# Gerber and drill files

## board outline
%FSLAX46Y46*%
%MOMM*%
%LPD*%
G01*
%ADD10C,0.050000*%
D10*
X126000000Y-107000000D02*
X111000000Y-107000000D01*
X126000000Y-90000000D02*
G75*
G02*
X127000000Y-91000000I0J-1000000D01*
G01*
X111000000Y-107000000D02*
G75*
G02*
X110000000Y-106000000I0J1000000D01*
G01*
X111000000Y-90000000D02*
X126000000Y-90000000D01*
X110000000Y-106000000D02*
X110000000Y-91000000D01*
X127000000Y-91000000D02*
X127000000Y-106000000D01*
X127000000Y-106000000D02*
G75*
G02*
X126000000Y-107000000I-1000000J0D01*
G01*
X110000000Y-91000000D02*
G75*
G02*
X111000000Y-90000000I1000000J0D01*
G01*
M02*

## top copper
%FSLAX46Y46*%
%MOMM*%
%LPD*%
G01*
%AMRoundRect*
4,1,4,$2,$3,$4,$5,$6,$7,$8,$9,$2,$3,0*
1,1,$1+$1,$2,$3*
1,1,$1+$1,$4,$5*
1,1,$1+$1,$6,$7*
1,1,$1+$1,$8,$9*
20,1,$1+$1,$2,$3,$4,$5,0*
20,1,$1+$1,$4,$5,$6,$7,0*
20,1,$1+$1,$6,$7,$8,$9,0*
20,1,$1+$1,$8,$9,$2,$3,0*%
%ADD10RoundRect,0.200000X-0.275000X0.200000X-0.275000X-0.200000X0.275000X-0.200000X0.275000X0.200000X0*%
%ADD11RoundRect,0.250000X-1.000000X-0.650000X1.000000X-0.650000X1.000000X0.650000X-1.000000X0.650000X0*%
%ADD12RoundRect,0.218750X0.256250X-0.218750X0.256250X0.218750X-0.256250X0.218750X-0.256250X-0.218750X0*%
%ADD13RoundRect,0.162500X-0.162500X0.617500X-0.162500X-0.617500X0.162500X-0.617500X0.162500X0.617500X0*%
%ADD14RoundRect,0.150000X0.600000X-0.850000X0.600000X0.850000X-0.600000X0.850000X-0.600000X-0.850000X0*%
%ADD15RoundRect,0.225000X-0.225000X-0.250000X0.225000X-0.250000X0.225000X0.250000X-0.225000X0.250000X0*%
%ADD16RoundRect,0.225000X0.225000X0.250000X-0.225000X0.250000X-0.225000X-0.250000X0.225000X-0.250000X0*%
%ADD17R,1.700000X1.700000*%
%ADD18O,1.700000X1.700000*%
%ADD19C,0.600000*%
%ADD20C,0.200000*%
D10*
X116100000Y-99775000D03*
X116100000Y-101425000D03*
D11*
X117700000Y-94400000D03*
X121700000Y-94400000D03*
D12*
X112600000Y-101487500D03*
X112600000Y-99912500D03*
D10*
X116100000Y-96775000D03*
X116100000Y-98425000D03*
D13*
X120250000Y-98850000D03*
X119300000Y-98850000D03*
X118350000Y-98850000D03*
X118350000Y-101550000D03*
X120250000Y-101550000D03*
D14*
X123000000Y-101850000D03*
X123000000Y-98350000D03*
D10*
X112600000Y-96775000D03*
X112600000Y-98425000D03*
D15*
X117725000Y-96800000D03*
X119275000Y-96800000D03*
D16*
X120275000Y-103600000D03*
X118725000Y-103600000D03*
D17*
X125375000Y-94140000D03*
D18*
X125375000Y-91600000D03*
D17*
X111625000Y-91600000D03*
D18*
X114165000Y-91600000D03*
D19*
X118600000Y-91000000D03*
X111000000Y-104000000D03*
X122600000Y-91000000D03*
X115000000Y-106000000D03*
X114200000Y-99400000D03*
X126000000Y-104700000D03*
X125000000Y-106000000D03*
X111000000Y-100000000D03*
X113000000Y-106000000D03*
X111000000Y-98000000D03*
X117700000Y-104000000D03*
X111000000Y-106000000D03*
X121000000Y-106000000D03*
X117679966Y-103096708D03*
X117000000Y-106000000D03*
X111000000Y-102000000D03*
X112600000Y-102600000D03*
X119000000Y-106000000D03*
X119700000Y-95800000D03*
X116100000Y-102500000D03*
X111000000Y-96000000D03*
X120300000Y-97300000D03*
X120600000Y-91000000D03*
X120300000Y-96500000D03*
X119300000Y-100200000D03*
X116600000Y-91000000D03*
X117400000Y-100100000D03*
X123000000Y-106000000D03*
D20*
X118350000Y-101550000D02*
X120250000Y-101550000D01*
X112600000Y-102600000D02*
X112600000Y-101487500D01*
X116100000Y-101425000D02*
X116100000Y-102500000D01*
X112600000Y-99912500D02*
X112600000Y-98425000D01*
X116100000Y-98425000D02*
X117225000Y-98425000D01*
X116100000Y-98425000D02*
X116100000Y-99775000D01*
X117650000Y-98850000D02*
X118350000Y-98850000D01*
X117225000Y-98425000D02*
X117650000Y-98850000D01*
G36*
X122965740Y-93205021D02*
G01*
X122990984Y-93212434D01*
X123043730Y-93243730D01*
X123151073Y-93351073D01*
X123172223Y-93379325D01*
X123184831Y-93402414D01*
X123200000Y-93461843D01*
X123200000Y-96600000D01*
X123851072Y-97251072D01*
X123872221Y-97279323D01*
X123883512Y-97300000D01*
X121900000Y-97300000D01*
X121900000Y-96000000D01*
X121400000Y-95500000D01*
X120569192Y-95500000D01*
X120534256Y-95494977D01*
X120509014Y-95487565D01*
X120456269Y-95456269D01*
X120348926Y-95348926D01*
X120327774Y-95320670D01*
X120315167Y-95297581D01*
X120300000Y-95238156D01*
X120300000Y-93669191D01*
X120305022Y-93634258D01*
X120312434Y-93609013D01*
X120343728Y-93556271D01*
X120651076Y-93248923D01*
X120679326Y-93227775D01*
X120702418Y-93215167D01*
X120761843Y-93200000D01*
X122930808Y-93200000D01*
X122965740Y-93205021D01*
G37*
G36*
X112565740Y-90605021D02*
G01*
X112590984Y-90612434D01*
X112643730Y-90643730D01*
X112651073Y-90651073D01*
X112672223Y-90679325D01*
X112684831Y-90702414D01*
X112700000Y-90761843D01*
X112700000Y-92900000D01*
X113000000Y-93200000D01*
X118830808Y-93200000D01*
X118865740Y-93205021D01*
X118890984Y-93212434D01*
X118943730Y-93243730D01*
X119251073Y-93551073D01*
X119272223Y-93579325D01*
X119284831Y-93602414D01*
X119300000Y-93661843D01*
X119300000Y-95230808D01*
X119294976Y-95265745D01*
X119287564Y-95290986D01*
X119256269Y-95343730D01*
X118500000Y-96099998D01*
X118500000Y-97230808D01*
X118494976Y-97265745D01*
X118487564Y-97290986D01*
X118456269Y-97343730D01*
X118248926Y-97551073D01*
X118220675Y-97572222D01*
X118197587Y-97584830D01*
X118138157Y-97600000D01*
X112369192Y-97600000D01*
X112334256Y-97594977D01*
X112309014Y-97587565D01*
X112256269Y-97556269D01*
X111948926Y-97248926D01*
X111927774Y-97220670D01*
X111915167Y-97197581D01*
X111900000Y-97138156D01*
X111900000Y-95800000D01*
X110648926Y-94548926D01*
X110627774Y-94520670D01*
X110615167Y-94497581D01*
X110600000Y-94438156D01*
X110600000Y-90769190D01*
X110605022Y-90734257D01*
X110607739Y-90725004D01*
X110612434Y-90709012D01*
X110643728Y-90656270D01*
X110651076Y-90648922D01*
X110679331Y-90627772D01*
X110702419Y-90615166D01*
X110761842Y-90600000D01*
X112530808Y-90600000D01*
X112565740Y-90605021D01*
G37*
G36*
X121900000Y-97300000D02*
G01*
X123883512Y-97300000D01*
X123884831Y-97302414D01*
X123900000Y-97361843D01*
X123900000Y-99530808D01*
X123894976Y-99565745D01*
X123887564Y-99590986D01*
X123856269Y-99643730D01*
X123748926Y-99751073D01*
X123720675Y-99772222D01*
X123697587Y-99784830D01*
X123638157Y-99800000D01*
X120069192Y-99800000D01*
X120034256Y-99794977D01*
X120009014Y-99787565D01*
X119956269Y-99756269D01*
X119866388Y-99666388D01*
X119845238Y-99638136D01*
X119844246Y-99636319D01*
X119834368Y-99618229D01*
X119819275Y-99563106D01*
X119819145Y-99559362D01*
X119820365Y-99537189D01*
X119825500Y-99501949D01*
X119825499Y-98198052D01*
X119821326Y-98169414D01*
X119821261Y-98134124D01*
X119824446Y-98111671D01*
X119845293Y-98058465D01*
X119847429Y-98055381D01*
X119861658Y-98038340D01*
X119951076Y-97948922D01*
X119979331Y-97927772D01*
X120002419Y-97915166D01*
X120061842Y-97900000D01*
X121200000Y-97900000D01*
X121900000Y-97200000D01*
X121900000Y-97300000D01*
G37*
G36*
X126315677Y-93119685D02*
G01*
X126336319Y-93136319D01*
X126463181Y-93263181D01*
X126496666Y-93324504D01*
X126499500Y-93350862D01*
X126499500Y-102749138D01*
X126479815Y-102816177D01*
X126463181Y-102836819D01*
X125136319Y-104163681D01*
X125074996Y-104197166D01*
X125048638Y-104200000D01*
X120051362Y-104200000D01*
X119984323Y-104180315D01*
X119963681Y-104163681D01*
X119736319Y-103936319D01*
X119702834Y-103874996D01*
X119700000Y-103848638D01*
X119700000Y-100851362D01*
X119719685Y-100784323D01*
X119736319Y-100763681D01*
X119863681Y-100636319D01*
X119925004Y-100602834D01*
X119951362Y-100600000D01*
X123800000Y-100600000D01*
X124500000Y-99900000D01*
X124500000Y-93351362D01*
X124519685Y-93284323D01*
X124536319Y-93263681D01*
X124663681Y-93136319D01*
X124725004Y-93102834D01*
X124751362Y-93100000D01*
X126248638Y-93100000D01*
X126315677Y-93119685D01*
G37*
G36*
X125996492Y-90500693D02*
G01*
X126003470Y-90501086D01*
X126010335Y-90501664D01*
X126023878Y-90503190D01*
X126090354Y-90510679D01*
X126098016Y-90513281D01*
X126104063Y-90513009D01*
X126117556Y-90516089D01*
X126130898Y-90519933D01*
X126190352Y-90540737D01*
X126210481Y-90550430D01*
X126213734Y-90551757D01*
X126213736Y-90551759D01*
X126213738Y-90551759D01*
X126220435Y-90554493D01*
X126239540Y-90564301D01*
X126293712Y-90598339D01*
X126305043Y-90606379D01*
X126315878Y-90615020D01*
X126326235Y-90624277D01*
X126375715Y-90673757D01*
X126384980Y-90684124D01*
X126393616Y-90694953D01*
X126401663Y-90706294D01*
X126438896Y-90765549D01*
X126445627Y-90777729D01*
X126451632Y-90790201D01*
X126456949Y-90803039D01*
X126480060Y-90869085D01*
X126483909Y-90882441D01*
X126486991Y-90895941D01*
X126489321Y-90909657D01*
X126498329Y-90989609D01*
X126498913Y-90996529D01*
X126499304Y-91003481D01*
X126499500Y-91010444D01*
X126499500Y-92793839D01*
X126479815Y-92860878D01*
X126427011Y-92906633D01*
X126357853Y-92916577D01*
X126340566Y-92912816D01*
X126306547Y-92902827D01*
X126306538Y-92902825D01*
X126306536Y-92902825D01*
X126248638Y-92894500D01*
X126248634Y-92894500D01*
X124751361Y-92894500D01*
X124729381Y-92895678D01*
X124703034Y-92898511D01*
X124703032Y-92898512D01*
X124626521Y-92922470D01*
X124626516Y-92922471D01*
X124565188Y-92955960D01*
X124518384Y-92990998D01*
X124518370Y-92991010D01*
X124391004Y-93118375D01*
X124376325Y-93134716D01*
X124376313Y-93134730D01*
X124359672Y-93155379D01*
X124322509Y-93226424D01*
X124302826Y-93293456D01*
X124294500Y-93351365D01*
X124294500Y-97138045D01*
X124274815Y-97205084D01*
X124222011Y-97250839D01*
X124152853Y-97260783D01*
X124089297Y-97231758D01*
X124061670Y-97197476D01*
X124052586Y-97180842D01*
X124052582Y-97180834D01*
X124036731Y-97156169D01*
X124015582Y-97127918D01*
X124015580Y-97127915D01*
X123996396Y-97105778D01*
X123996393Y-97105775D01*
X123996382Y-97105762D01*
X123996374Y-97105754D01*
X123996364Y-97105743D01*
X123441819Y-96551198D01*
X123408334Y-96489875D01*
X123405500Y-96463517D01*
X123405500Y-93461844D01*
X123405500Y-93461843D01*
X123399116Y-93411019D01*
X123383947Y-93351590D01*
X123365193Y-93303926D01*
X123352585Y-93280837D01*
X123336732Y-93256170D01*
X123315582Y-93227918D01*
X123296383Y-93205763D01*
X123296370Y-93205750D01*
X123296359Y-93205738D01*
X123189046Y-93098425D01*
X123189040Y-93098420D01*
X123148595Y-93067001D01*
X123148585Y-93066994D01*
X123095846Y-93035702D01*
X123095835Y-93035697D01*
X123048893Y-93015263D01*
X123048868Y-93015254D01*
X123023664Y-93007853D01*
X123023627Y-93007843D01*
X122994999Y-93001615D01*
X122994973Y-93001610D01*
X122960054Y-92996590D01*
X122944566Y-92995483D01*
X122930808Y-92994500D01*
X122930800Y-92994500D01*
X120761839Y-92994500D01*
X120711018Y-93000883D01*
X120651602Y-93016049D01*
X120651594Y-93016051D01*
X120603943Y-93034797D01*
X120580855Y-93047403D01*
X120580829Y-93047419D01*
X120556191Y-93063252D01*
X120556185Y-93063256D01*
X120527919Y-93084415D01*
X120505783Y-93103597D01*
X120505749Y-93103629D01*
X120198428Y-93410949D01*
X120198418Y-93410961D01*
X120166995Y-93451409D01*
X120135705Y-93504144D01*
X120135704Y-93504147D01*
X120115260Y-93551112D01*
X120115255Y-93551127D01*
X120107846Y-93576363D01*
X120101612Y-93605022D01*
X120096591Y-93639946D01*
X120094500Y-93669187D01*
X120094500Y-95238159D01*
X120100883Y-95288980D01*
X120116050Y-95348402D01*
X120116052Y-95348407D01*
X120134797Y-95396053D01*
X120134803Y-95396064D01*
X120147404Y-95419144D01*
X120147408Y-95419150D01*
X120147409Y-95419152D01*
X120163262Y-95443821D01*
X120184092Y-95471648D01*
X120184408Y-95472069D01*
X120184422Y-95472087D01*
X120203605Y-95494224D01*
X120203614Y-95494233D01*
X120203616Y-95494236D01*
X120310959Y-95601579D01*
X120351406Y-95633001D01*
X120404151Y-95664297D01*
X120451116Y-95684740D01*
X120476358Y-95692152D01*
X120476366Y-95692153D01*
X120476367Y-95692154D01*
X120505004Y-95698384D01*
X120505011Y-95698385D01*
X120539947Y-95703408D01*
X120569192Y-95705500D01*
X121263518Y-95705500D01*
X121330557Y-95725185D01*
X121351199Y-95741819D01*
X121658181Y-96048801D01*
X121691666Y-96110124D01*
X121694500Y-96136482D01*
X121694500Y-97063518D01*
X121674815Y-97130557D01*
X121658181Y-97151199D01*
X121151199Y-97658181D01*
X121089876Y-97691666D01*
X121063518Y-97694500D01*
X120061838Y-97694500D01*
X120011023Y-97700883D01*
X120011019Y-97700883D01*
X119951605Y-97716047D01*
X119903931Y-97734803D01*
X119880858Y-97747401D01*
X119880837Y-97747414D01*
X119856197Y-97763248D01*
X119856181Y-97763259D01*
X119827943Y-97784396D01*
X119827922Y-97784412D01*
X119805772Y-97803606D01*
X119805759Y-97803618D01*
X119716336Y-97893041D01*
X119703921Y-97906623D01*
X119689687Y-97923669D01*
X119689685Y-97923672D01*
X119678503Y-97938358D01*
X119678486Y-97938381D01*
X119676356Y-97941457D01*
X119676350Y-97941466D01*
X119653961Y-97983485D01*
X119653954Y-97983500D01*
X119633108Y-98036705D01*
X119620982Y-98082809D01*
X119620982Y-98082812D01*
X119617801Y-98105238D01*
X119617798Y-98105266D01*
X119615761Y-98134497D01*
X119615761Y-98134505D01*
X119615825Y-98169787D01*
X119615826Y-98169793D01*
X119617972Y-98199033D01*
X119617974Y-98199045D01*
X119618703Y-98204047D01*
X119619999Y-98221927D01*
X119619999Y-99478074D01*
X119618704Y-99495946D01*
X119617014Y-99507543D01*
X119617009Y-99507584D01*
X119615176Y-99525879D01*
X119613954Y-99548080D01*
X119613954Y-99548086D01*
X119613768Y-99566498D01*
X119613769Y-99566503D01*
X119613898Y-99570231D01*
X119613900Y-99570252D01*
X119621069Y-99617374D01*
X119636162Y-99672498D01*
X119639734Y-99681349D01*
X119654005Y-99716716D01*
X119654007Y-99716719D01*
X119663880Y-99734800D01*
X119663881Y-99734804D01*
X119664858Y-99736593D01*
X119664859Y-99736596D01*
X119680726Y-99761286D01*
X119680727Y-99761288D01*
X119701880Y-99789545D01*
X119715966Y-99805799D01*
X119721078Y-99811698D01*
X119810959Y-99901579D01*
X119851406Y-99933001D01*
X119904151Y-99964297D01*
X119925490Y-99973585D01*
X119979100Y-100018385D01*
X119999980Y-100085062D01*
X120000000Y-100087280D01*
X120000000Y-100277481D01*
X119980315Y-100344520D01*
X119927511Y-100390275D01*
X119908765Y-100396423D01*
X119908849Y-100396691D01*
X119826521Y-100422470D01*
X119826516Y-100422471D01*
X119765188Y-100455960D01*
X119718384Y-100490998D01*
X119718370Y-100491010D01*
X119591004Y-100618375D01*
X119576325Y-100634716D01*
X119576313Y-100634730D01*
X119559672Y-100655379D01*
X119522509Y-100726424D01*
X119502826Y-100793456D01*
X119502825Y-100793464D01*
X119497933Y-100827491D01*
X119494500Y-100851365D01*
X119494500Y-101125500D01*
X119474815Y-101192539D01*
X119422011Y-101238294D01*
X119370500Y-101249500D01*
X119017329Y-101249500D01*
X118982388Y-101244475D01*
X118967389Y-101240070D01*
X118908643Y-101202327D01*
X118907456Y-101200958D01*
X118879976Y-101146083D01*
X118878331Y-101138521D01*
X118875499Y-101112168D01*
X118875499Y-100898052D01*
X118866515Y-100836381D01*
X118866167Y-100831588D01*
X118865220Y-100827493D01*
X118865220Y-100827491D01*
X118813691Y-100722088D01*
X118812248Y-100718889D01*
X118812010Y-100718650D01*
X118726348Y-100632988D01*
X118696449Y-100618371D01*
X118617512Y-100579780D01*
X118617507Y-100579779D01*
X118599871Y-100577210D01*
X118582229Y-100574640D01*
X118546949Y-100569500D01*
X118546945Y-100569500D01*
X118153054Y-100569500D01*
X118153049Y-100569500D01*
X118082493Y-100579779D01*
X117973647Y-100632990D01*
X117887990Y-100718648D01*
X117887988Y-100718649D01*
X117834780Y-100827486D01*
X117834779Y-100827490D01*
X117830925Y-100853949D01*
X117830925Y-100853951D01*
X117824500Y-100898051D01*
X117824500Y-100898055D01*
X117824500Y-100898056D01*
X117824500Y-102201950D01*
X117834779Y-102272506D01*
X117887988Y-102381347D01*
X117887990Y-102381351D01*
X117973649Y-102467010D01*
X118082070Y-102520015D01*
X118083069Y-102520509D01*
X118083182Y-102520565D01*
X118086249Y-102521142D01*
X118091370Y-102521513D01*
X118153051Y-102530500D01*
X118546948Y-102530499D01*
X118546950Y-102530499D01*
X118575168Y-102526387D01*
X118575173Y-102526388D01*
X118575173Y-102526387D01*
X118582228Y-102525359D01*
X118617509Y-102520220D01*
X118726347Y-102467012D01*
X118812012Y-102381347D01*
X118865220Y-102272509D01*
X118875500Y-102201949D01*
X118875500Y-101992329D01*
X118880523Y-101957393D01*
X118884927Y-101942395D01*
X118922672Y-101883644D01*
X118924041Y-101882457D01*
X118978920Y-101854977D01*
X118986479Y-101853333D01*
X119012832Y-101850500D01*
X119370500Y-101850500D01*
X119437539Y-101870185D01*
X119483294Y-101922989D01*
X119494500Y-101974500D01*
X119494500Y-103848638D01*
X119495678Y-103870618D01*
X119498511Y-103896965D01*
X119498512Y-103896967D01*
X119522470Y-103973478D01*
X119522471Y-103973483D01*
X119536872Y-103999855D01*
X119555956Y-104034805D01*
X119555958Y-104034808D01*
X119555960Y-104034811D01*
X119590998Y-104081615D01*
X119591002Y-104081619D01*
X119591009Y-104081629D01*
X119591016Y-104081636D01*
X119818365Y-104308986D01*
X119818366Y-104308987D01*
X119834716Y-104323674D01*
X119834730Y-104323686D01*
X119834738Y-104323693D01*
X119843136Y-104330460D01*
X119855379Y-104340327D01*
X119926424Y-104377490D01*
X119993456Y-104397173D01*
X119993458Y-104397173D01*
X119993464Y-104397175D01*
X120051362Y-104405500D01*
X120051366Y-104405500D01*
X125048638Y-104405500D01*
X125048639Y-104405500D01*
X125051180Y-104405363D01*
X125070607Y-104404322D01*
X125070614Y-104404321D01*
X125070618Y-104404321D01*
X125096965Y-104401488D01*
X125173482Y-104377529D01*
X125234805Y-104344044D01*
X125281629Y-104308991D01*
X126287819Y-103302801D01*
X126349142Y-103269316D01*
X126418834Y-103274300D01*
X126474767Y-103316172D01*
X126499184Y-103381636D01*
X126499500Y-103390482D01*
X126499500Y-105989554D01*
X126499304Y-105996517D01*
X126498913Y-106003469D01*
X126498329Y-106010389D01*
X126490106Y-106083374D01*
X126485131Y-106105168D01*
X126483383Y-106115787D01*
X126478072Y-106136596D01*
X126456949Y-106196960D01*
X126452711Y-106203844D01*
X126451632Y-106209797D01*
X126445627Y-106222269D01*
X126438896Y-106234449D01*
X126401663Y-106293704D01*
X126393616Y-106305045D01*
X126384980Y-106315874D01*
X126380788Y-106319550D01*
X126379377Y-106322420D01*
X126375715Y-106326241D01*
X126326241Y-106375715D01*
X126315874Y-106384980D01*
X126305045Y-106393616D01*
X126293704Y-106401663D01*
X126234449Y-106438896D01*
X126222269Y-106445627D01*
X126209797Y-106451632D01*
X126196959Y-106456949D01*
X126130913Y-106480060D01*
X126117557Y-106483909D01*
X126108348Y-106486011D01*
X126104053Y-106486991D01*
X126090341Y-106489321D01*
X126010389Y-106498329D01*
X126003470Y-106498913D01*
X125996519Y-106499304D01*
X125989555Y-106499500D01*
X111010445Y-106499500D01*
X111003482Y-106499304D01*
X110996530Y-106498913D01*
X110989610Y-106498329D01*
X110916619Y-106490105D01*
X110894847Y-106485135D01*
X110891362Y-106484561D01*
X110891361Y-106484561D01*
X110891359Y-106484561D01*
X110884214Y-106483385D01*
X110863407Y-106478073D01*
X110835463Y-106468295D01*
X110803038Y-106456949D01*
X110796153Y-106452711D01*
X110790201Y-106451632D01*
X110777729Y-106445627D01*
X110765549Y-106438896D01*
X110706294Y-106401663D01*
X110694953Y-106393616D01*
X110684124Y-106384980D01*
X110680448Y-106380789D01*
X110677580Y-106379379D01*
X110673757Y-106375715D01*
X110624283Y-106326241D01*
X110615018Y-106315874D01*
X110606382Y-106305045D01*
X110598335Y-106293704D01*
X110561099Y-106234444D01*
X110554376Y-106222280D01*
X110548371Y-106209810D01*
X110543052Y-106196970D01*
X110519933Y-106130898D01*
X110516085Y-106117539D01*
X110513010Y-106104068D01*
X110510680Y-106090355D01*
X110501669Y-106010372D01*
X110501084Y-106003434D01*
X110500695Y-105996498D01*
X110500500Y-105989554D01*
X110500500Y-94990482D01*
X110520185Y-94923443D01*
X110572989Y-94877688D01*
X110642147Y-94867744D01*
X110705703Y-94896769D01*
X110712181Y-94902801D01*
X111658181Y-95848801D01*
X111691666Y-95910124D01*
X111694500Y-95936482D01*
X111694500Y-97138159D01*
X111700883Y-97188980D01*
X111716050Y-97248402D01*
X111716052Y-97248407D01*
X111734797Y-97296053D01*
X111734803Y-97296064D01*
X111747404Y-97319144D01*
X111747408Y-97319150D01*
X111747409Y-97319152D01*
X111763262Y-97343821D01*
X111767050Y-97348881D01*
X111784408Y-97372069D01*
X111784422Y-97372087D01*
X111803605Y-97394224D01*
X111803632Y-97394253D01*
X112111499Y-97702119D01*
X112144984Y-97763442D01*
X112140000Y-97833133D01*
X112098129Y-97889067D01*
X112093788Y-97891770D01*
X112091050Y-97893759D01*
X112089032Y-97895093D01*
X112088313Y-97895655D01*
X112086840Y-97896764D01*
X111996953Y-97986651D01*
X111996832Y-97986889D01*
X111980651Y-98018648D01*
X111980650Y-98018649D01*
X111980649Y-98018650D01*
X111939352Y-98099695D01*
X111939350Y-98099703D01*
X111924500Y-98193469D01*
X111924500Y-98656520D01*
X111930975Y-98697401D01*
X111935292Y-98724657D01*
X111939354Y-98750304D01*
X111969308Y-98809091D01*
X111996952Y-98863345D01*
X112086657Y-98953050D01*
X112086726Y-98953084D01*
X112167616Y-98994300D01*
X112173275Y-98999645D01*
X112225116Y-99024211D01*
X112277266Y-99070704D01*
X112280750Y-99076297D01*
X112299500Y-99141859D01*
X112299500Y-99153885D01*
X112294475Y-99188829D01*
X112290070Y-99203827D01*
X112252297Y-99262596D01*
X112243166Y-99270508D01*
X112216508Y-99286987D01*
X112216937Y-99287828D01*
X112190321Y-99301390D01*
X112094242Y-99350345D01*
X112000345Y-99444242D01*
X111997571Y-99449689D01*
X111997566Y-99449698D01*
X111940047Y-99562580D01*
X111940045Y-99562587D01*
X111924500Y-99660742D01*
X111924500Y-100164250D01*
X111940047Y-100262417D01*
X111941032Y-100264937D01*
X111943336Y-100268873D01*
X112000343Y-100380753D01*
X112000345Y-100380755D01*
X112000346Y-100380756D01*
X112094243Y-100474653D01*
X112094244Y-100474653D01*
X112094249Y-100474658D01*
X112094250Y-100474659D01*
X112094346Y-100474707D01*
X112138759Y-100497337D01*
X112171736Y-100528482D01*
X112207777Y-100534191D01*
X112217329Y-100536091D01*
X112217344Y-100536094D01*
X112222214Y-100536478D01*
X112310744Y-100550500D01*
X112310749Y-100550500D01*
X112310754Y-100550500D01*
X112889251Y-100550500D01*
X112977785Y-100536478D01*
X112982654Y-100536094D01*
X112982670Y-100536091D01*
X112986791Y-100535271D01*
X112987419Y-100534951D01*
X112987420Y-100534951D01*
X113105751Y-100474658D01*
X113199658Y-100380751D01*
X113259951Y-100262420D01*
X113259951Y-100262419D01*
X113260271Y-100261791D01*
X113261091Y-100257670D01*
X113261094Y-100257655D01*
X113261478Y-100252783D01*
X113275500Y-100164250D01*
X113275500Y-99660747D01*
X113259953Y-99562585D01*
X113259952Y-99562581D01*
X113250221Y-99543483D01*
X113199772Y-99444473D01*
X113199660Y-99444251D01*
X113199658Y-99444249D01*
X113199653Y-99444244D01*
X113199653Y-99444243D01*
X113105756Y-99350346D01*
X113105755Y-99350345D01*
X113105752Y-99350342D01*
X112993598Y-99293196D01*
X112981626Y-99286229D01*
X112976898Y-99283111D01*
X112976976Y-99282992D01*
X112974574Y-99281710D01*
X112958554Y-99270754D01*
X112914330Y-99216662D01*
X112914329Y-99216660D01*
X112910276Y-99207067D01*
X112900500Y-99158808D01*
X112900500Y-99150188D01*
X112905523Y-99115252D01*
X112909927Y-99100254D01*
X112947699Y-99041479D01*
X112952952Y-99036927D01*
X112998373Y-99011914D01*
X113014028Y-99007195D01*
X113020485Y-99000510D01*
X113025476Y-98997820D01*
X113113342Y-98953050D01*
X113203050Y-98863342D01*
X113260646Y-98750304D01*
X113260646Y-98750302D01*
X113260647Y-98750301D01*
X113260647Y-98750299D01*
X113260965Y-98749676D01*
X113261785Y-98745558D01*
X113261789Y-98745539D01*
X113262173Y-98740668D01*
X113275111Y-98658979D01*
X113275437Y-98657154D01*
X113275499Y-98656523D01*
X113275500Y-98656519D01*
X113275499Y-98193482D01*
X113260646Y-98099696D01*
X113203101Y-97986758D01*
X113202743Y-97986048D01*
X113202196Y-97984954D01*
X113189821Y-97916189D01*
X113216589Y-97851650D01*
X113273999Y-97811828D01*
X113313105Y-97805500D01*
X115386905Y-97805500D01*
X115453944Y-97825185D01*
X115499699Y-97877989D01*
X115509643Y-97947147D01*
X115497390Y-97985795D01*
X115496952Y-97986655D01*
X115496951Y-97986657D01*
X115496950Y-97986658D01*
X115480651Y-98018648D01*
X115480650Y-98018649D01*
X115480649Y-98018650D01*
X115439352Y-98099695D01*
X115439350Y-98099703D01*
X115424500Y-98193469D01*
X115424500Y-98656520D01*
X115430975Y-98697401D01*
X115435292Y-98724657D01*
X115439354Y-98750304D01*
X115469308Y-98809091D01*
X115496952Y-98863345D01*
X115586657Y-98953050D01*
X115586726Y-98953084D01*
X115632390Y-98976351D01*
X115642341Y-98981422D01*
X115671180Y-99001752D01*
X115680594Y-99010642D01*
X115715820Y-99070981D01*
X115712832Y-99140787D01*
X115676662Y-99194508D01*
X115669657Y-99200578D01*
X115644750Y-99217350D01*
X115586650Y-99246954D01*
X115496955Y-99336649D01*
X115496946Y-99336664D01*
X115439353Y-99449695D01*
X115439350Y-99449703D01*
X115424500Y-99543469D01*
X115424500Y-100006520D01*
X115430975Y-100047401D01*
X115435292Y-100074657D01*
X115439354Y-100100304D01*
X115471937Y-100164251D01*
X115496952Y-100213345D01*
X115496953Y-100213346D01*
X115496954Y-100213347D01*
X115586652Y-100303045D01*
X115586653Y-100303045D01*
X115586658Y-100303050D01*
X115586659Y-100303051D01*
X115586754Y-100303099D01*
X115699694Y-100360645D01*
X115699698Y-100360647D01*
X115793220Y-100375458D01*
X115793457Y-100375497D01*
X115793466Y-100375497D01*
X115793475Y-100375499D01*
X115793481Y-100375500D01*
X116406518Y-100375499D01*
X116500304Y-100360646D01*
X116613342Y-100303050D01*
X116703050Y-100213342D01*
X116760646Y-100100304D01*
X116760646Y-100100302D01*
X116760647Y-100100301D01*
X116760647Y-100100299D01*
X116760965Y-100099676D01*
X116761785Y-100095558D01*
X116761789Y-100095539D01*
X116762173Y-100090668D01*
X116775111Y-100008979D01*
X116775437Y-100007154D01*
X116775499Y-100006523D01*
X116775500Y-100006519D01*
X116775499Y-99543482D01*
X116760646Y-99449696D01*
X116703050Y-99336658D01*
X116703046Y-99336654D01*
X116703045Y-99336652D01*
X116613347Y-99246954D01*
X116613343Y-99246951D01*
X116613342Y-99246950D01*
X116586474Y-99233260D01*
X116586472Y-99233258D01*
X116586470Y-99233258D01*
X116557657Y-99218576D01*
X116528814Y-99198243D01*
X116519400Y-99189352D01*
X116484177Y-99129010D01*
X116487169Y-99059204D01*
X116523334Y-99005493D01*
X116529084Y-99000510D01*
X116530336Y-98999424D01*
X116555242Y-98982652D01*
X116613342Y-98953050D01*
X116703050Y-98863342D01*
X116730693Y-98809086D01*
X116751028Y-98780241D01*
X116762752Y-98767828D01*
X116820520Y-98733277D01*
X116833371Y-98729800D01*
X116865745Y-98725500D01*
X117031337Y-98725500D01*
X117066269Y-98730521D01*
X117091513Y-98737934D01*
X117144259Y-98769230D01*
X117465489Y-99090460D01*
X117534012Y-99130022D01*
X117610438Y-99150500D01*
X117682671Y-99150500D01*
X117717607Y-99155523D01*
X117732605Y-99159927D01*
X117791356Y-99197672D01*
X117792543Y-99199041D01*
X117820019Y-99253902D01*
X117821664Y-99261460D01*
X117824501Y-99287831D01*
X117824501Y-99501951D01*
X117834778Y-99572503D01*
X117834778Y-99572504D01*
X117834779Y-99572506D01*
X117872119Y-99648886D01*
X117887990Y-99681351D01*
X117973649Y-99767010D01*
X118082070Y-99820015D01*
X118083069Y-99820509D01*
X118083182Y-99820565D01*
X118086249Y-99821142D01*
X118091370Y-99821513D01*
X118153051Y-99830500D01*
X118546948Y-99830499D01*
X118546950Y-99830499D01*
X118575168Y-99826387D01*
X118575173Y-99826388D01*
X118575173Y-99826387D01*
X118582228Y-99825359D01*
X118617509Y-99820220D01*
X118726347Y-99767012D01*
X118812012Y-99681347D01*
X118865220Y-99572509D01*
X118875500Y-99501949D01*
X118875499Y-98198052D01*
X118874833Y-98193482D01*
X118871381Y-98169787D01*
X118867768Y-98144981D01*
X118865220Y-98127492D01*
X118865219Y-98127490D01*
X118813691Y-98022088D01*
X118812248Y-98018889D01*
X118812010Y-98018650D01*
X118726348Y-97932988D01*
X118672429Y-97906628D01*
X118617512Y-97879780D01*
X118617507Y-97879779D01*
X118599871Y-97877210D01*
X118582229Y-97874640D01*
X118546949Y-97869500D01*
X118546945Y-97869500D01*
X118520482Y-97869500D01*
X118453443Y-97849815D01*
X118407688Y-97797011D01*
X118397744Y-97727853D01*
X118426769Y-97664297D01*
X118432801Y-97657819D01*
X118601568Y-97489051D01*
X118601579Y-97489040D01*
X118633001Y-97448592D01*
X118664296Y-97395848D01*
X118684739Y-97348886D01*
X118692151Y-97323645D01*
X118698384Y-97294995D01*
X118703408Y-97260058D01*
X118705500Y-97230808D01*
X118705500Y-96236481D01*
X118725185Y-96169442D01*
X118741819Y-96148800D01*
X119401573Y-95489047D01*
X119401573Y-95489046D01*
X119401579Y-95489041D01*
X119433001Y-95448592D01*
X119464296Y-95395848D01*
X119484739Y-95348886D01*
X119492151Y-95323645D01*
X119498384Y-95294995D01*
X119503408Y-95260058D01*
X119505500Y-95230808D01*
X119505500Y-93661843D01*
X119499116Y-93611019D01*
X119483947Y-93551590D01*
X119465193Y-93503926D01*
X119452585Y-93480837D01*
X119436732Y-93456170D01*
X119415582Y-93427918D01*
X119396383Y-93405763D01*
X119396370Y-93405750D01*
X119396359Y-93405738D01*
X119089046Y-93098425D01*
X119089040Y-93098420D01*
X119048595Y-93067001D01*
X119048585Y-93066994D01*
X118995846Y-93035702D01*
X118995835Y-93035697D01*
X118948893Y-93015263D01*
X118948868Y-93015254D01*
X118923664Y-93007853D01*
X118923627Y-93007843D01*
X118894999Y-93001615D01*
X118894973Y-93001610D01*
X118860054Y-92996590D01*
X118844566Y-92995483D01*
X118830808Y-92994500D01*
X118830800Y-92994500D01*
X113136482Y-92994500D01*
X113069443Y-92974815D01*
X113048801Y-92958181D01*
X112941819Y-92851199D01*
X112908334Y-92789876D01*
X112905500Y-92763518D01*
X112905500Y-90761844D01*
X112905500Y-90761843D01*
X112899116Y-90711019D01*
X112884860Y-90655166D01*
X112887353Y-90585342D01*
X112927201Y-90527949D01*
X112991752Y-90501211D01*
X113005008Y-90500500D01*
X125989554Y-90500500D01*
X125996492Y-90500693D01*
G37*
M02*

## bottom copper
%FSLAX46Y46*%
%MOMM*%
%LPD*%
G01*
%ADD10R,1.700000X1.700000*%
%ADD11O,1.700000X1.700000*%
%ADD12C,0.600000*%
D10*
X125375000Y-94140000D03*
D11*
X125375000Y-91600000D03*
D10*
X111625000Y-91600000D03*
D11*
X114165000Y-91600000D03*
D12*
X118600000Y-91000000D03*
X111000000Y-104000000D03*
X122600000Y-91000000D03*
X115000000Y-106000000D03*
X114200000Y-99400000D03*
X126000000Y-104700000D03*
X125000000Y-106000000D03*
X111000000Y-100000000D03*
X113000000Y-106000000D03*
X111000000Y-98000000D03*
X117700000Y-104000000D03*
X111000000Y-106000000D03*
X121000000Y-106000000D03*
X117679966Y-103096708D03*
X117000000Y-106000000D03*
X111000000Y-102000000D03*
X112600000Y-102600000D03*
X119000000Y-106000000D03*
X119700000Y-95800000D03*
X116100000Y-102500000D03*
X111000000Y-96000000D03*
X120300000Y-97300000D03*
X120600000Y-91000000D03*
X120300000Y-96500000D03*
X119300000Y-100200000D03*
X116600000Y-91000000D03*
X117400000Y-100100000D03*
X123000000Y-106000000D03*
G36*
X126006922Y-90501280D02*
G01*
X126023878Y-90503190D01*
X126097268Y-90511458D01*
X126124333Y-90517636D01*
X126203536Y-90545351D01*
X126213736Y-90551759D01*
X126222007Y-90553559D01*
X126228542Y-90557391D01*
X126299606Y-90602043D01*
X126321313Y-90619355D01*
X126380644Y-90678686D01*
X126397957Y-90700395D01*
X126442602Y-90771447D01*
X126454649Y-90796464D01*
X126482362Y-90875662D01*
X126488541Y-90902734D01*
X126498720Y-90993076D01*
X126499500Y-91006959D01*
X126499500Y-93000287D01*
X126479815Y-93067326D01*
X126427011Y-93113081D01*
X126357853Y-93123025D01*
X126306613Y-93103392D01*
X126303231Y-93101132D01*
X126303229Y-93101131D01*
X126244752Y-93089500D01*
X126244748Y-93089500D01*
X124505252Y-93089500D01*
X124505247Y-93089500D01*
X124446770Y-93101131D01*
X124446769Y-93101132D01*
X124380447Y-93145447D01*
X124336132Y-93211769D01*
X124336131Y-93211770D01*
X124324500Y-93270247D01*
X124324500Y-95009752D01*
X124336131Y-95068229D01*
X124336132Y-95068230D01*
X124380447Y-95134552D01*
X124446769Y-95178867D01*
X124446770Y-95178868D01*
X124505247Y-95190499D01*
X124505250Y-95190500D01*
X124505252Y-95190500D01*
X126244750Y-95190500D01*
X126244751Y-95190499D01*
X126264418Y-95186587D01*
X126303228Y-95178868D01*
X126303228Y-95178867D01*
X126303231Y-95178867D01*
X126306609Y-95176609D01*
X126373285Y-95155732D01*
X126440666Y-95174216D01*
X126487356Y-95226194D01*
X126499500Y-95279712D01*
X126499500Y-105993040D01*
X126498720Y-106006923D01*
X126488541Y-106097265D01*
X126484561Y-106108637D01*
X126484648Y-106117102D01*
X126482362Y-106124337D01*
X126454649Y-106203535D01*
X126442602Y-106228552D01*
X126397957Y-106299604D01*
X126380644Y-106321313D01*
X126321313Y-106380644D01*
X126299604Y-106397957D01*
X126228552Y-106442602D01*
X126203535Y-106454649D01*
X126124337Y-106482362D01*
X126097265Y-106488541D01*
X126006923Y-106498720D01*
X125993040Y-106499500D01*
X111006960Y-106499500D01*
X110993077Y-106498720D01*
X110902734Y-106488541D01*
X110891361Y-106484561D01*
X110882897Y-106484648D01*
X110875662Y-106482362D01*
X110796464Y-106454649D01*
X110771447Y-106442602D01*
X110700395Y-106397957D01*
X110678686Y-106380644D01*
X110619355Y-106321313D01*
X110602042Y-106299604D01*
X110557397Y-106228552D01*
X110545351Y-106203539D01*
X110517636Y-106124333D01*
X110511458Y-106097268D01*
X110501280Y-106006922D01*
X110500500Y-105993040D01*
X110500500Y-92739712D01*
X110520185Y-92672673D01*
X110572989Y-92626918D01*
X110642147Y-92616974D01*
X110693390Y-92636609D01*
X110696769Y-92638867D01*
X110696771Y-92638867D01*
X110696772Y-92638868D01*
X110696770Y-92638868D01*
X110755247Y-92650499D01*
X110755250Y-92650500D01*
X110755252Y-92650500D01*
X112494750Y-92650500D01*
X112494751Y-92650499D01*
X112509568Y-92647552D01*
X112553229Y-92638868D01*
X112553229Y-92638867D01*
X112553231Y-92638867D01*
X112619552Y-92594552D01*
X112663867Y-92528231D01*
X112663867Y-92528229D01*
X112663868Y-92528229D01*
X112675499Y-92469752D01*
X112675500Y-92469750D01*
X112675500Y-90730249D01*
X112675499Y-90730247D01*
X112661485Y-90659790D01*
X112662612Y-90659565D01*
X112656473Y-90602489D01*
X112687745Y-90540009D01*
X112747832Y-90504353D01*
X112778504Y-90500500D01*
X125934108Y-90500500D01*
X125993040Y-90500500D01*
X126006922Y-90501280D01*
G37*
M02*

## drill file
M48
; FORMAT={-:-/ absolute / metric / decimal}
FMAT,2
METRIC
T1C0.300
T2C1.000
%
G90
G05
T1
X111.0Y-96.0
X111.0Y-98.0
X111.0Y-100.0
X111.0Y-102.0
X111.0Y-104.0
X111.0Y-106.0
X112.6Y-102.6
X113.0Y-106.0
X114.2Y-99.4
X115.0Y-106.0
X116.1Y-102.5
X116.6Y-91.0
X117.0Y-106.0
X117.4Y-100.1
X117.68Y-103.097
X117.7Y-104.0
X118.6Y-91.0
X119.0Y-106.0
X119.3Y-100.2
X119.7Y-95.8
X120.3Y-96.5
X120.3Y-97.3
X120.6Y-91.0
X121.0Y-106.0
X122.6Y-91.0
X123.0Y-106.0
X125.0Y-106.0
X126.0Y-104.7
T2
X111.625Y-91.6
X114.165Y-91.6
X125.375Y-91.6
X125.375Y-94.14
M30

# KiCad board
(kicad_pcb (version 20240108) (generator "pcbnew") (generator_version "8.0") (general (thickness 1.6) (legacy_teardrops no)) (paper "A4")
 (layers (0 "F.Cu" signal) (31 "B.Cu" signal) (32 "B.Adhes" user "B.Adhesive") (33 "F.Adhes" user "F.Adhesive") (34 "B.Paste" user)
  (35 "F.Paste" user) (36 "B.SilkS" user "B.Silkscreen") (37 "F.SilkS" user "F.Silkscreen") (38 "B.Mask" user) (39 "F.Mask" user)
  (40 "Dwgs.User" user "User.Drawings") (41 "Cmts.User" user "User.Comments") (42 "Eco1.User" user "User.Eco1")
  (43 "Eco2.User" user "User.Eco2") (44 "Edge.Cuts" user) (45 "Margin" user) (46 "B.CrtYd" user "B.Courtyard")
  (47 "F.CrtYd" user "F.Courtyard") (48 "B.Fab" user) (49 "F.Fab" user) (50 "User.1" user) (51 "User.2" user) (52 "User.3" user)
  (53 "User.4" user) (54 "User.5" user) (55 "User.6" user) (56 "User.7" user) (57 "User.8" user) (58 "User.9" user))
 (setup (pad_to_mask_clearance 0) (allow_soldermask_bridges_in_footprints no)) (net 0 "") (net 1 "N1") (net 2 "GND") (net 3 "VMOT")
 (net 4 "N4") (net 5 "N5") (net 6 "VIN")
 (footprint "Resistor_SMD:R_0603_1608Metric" (layer "F.Cu") (at 116.1 100.6 -90)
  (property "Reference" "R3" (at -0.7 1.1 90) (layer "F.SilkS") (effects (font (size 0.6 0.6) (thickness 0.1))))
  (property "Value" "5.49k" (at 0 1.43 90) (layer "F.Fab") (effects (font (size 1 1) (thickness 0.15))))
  (pad "1" smd roundrect (at -0.825 0 270) (size 0.8 0.95) (layers "F.Cu" "F.Paste" "F.Mask") (roundrect_rratio 0.25) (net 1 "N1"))
  (pad "2" smd roundrect (at 0.825 0 270) (size 0.8 0.95) (layers "F.Cu" "F.Paste" "F.Mask") (roundrect_rratio 0.25) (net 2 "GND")))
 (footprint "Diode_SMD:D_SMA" (layer "F.Cu") (at 119.7 94.4)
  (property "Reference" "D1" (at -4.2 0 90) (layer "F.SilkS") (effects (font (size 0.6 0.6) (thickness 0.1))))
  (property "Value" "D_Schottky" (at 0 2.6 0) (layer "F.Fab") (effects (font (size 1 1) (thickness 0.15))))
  (pad "1" smd roundrect (at -2 0) (size 2.5 1.8) (layers "F.Cu" "F.Paste" "F.Mask") (roundrect_rratio 0.1388888889) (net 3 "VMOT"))
  (pad "2" smd roundrect (at 2 0) (size 2.5 1.8) (layers "F.Cu" "F.Paste" "F.Mask") (roundrect_rratio 0.1388888889) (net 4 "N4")))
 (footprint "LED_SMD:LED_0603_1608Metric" (layer "F.Cu") (at 112.6 100.7 90)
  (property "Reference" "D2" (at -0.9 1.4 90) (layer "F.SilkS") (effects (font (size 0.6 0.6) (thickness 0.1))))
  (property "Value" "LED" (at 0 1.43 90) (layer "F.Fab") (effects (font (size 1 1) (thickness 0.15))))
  (pad "1" smd roundrect (at -0.7875 0 90) (size 0.875 0.95) (layers "F.Cu" "F.Paste" "F.Mask") (roundrect_rratio 0.25) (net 2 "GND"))
  (pad "2" smd roundrect (at 0.7875 0 90) (size 0.875 0.95) (layers "F.Cu" "F.Paste" "F.Mask") (roundrect_rratio 0.25) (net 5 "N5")))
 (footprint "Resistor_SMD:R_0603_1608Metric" (layer "F.Cu") (at 116.1 97.6 -90)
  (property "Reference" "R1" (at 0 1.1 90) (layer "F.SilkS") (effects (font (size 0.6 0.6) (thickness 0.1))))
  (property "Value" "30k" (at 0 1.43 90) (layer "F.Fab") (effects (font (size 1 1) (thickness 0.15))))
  (pad "1" smd roundrect (at -0.825 0 270) (size 0.8 0.95) (layers "F.Cu" "F.Paste" "F.Mask") (roundrect_rratio 0.25) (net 3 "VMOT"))
  (pad "2" smd roundrect (at 0.825 0 270) (size 0.8 0.95) (layers "F.Cu" "F.Paste" "F.Mask") (roundrect_rratio 0.25) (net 1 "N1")))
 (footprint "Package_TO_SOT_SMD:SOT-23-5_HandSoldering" (layer "F.Cu") (at 119.3 100.2 -90)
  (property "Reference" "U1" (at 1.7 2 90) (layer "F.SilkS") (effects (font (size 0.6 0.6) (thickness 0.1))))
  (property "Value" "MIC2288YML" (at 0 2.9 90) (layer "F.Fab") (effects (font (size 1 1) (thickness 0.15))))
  (pad "1" smd roundrect (at -1.35 -0.95 270) (size 1.56 0.65) (layers "F.Cu" "F.Paste" "F.Mask") (roundrect_rratio 0.25) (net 4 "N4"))
  (pad "2" smd roundrect (at -1.35 0 270) (size 1.56 0.65) (layers "F.Cu" "F.Paste" "F.Mask") (roundrect_rratio 0.25) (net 2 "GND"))
  (pad "3" smd roundrect (at -1.35 0.95 270) (size 1.56 0.65) (layers "F.Cu" "F.Paste" "F.Mask") (roundrect_rratio 0.25) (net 1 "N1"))
  (pad "4" smd roundrect (at 1.35 0.95 270) (size 1.56 0.65) (layers "F.Cu" "F.Paste" "F.Mask") (roundrect_rratio 0.25) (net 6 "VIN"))
  (pad "5" smd roundrect (at 1.35 -0.95 270) (size 1.56 0.65) (layers "F.Cu" "F.Paste" "F.Mask") (roundrect_rratio 0.25) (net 6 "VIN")))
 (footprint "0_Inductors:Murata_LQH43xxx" (layer "F.Cu") (at 123 100.1 90)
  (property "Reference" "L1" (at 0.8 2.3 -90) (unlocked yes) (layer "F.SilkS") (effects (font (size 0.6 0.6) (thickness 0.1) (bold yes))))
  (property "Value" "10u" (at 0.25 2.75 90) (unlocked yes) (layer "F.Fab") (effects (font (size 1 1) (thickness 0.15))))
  (pad "1" smd roundrect (at -1.75 0 90) (size 2 1.5) (layers "F.Cu" "F.Paste" "F.Mask") (roundrect_rratio 0.1) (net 6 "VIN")
   (thermal_bridge_angle 45))
  (pad "2" smd roundrect (at 1.75 0 90) (size 2 1.5) (layers "F.Cu" "F.Paste" "F.Mask") (roundrect_rratio 0.1) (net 4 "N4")
   (thermal_bridge_angle 45)))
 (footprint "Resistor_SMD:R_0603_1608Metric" (layer "F.Cu") (at 112.6 97.6 -90)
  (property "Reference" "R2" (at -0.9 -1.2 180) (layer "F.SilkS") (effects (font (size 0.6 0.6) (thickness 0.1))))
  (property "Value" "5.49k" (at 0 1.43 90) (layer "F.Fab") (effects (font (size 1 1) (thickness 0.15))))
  (pad "1" smd roundrect (at -0.825 0 270) (size 0.8 0.95) (layers "F.Cu" "F.Paste" "F.Mask") (roundrect_rratio 0.25) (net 3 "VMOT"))
  (pad "2" smd roundrect (at 0.825 0 270) (size 0.8 0.95) (layers "F.Cu" "F.Paste" "F.Mask") (roundrect_rratio 0.25) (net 5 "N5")))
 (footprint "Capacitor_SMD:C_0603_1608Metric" (layer "F.Cu") (at 118.5 96.8)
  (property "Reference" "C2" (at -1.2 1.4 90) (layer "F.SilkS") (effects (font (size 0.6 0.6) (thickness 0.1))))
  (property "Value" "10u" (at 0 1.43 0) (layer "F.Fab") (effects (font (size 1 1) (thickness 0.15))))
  (pad "1" smd roundrect (at -0.775 0) (size 0.9 0.95) (layers "F.Cu" "F.Paste" "F.Mask") (roundrect_rratio 0.25) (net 3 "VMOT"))
  (pad "2" smd roundrect (at 0.775 0) (size 0.9 0.95) (layers "F.Cu" "F.Paste" "F.Mask") (roundrect_rratio 0.25) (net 2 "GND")))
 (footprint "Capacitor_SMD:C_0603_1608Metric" (layer "F.Cu") (at 119.5 103.6 180)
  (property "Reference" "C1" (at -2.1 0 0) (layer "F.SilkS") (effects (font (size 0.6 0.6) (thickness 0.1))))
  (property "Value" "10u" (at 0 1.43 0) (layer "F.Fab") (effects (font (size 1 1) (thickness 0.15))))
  (pad "1" smd roundrect (at -0.775 0 180) (size 0.9 0.95) (layers "F.Cu" "F.Paste" "F.Mask") (roundrect_rratio 0.25) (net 6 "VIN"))
  (pad "2" smd roundrect (at 0.775 0 180) (size 0.9 0.95) (layers "F.Cu" "F.Paste" "F.Mask") (roundrect_rratio 0.25) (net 2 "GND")))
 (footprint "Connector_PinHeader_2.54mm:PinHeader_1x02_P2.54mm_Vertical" (layer "B.Cu") (at 125.375 94.14)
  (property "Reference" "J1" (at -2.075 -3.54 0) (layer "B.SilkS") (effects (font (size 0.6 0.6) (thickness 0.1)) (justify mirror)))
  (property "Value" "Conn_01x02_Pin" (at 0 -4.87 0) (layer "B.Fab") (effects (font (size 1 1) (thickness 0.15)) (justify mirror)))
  (pad "1" thru_hole rect (at 0 0) (size 1.7 1.7) (drill 1) (layers "*.Cu" "*.Mask") (remove_unused_layers no) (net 6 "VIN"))
  (pad "2" thru_hole oval (at 0 -2.54) (size 1.7 1.7) (drill 1) (layers "*.Cu" "*.Mask") (remove_unused_layers no) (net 2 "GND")))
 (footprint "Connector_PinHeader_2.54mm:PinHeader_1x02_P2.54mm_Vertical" (layer "B.Cu") (at 111.625 91.6 -90)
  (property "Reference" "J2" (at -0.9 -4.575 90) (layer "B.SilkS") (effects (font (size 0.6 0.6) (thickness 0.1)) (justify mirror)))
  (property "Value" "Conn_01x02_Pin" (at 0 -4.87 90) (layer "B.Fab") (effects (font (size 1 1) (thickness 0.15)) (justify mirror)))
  (pad "1" thru_hole rect (at 0 0 270) (size 1.7 1.7) (drill 1) (layers "*.Cu" "*.Mask") (remove_unused_layers no) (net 3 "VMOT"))
  (pad "2" thru_hole oval (at 0 -2.54 270) (size 1.7 1.7) (drill 1) (layers "*.Cu" "*.Mask") (remove_unused_layers no) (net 2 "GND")))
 (gr_line (start 126 107) (end 111 107) (stroke (width 0.05) (type default)) (layer "Edge.Cuts"))
 (gr_arc (start 126 90) (mid 126.707107 90.292893) (end 127 91) (stroke (width 0.05) (type default)) (layer "Edge.Cuts"))
 (gr_arc (start 111 107) (mid 110.292893 106.707107) (end 110 106) (stroke (width 0.05) (type default)) (layer "Edge.Cuts"))
 (gr_line (start 111 90) (end 126 90) (stroke (width 0.05) (type default)) (layer "Edge.Cuts"))
 (gr_line (start 110 106) (end 110 91) (stroke (width 0.05) (type default)) (layer "Edge.Cuts"))
 (gr_line (start 127 91) (end 127 106) (stroke (width 0.05) (type default)) (layer "Edge.Cuts"))
 (gr_arc (start 127 106) (mid 126.707107 106.707107) (end 126 107) (stroke (width 0.05) (type default)) (layer "Edge.Cuts"))
 (gr_arc (start 110 91) (mid 110.292893 90.292893) (end 111 90) (stroke (width 0.05) (type default)) (layer "Edge.Cuts"))
 (segment (start 118.35 101.55) (end 120.25 101.55) (width 0.2) (layer "F.Cu") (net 6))
 (segment (start 112.6 102.6) (end 112.6 101.4875) (width 0.2) (layer "F.Cu") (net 2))
 (segment (start 116.1 101.425) (end 116.1 102.5) (width 0.2) (layer "F.Cu") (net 2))
 (via (at 118.6 91) (size 0.6) (drill 0.3) (layers "F.Cu" "B.Cu") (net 2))
 (via (at 111 104) (size 0.6) (drill 0.3) (layers "F.Cu" "B.Cu") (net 2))
 (via (at 122.6 91) (size 0.6) (drill 0.3) (layers "F.Cu" "B.Cu") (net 2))
 (via (at 115 106) (size 0.6) (drill 0.3) (layers "F.Cu" "B.Cu") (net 2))
 (via (at 114.2 99.4) (size 0.6) (drill 0.3) (layers "F.Cu" "B.Cu") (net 2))
 (via (at 126 104.7) (size 0.6) (drill 0.3) (layers "F.Cu" "B.Cu") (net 2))
 (via (at 125 106) (size 0.6) (drill 0.3) (layers "F.Cu" "B.Cu") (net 2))
 (via (at 111 100) (size 0.6) (drill 0.3) (layers "F.Cu" "B.Cu") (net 2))
 (via (at 113 106) (size 0.6) (drill 0.3) (layers "F.Cu" "B.Cu") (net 2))
 (via (at 111 98) (size 0.6) (drill 0.3) (layers "F.Cu" "B.Cu") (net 2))
 (via (at 117.7 104) (size 0.6) (drill 0.3) (layers "F.Cu" "B.Cu") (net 2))
 (via (at 111 106) (size 0.6) (drill 0.3) (layers "F.Cu" "B.Cu") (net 2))
 (via (at 121 106) (size 0.6) (drill 0.3) (layers "F.Cu" "B.Cu") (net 2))
 (via (at 117.679966 103.096708) (size 0.6) (drill 0.3) (layers "F.Cu" "B.Cu") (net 2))
 (via (at 117 106) (size 0.6) (drill 0.3) (layers "F.Cu" "B.Cu") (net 2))
 (via (at 111 102) (size 0.6) (drill 0.3) (layers "F.Cu" "B.Cu") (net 2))
 (via (at 112.6 102.6) (size 0.6) (drill 0.3) (layers "F.Cu" "B.Cu") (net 2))
 (via (at 119 106) (size 0.6) (drill 0.3) (layers "F.Cu" "B.Cu") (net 2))
 (via (at 119.7 95.8) (size 0.6) (drill 0.3) (layers "F.Cu" "B.Cu") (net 2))
 (via (at 116.1 102.5) (size 0.6) (drill 0.3) (layers "F.Cu" "B.Cu") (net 2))
 (via (at 111 96) (size 0.6) (drill 0.3) (layers "F.Cu" "B.Cu") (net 2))
 (via (at 120.3 97.3) (size 0.6) (drill 0.3) (layers "F.Cu" "B.Cu") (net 2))
 (via (at 120.6 91) (size 0.6) (drill 0.3) (layers "F.Cu" "B.Cu") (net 2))
 (via (at 120.3 96.5) (size 0.6) (drill 0.3) (layers "F.Cu" "B.Cu") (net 2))
 (via (at 119.3 100.2) (size 0.6) (drill 0.3) (layers "F.Cu" "B.Cu") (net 2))
 (via (at 116.6 91) (size 0.6) (drill 0.3) (layers "F.Cu" "B.Cu") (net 2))
 (via (at 117.4 100.1) (size 0.6) (drill 0.3) (layers "F.Cu" "B.Cu") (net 2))
 (via (at 123 106) (size 0.6) (drill 0.3) (layers "F.Cu" "B.Cu") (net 2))
 (segment (start 112.6 99.9125) (end 112.6 98.425) (width 0.2) (layer "F.Cu") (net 5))
 (segment (start 116.1 98.425) (end 117.225 98.425) (width 0.2) (layer "F.Cu") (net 1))
 (segment (start 116.1 98.425) (end 116.1 99.775) (width 0.2) (layer "F.Cu") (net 1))
 (segment (start 117.65 98.85) (end 118.35 98.85) (width 0.2) (layer "F.Cu") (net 1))
 (segment (start 117.225 98.425) (end 117.65 98.85) (width 0.2) (layer "F.Cu") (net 1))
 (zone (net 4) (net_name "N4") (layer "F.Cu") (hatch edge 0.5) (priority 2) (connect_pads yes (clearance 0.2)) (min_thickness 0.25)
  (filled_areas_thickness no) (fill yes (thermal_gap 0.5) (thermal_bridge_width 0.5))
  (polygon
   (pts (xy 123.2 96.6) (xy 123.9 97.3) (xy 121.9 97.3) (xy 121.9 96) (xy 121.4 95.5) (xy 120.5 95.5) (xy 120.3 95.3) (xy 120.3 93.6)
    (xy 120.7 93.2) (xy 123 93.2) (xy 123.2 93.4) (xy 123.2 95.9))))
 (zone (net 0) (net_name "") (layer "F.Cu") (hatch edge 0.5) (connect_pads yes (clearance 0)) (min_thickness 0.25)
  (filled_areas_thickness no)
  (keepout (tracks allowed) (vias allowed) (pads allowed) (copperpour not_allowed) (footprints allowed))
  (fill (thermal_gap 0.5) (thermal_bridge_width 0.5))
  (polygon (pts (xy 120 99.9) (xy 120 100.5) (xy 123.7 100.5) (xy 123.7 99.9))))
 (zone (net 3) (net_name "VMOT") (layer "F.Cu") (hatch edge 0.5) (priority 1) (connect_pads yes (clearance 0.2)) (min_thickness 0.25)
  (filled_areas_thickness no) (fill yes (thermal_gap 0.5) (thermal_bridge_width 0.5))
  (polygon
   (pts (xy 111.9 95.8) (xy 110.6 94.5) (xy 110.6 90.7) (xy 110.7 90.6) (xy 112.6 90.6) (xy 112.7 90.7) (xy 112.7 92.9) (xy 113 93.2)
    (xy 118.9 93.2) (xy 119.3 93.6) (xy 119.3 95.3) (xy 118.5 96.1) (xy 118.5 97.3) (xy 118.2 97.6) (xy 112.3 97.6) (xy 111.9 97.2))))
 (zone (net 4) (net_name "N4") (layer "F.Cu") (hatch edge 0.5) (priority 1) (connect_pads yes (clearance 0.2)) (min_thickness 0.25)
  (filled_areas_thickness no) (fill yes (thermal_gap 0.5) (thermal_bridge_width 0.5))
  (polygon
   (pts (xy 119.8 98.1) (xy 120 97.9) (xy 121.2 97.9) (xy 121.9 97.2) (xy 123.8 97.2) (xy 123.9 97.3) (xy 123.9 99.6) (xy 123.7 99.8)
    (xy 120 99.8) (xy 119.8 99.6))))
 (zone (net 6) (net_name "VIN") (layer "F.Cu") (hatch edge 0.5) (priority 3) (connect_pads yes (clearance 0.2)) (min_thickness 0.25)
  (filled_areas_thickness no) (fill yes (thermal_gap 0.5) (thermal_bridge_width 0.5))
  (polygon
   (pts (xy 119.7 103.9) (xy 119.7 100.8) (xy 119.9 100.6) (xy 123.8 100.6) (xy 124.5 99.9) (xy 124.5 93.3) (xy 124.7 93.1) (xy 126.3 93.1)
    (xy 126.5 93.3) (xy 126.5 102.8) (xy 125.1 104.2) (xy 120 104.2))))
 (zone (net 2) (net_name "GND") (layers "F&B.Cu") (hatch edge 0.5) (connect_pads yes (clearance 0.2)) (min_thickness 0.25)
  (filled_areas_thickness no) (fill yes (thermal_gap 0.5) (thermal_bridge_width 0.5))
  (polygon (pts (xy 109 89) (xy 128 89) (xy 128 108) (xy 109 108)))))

